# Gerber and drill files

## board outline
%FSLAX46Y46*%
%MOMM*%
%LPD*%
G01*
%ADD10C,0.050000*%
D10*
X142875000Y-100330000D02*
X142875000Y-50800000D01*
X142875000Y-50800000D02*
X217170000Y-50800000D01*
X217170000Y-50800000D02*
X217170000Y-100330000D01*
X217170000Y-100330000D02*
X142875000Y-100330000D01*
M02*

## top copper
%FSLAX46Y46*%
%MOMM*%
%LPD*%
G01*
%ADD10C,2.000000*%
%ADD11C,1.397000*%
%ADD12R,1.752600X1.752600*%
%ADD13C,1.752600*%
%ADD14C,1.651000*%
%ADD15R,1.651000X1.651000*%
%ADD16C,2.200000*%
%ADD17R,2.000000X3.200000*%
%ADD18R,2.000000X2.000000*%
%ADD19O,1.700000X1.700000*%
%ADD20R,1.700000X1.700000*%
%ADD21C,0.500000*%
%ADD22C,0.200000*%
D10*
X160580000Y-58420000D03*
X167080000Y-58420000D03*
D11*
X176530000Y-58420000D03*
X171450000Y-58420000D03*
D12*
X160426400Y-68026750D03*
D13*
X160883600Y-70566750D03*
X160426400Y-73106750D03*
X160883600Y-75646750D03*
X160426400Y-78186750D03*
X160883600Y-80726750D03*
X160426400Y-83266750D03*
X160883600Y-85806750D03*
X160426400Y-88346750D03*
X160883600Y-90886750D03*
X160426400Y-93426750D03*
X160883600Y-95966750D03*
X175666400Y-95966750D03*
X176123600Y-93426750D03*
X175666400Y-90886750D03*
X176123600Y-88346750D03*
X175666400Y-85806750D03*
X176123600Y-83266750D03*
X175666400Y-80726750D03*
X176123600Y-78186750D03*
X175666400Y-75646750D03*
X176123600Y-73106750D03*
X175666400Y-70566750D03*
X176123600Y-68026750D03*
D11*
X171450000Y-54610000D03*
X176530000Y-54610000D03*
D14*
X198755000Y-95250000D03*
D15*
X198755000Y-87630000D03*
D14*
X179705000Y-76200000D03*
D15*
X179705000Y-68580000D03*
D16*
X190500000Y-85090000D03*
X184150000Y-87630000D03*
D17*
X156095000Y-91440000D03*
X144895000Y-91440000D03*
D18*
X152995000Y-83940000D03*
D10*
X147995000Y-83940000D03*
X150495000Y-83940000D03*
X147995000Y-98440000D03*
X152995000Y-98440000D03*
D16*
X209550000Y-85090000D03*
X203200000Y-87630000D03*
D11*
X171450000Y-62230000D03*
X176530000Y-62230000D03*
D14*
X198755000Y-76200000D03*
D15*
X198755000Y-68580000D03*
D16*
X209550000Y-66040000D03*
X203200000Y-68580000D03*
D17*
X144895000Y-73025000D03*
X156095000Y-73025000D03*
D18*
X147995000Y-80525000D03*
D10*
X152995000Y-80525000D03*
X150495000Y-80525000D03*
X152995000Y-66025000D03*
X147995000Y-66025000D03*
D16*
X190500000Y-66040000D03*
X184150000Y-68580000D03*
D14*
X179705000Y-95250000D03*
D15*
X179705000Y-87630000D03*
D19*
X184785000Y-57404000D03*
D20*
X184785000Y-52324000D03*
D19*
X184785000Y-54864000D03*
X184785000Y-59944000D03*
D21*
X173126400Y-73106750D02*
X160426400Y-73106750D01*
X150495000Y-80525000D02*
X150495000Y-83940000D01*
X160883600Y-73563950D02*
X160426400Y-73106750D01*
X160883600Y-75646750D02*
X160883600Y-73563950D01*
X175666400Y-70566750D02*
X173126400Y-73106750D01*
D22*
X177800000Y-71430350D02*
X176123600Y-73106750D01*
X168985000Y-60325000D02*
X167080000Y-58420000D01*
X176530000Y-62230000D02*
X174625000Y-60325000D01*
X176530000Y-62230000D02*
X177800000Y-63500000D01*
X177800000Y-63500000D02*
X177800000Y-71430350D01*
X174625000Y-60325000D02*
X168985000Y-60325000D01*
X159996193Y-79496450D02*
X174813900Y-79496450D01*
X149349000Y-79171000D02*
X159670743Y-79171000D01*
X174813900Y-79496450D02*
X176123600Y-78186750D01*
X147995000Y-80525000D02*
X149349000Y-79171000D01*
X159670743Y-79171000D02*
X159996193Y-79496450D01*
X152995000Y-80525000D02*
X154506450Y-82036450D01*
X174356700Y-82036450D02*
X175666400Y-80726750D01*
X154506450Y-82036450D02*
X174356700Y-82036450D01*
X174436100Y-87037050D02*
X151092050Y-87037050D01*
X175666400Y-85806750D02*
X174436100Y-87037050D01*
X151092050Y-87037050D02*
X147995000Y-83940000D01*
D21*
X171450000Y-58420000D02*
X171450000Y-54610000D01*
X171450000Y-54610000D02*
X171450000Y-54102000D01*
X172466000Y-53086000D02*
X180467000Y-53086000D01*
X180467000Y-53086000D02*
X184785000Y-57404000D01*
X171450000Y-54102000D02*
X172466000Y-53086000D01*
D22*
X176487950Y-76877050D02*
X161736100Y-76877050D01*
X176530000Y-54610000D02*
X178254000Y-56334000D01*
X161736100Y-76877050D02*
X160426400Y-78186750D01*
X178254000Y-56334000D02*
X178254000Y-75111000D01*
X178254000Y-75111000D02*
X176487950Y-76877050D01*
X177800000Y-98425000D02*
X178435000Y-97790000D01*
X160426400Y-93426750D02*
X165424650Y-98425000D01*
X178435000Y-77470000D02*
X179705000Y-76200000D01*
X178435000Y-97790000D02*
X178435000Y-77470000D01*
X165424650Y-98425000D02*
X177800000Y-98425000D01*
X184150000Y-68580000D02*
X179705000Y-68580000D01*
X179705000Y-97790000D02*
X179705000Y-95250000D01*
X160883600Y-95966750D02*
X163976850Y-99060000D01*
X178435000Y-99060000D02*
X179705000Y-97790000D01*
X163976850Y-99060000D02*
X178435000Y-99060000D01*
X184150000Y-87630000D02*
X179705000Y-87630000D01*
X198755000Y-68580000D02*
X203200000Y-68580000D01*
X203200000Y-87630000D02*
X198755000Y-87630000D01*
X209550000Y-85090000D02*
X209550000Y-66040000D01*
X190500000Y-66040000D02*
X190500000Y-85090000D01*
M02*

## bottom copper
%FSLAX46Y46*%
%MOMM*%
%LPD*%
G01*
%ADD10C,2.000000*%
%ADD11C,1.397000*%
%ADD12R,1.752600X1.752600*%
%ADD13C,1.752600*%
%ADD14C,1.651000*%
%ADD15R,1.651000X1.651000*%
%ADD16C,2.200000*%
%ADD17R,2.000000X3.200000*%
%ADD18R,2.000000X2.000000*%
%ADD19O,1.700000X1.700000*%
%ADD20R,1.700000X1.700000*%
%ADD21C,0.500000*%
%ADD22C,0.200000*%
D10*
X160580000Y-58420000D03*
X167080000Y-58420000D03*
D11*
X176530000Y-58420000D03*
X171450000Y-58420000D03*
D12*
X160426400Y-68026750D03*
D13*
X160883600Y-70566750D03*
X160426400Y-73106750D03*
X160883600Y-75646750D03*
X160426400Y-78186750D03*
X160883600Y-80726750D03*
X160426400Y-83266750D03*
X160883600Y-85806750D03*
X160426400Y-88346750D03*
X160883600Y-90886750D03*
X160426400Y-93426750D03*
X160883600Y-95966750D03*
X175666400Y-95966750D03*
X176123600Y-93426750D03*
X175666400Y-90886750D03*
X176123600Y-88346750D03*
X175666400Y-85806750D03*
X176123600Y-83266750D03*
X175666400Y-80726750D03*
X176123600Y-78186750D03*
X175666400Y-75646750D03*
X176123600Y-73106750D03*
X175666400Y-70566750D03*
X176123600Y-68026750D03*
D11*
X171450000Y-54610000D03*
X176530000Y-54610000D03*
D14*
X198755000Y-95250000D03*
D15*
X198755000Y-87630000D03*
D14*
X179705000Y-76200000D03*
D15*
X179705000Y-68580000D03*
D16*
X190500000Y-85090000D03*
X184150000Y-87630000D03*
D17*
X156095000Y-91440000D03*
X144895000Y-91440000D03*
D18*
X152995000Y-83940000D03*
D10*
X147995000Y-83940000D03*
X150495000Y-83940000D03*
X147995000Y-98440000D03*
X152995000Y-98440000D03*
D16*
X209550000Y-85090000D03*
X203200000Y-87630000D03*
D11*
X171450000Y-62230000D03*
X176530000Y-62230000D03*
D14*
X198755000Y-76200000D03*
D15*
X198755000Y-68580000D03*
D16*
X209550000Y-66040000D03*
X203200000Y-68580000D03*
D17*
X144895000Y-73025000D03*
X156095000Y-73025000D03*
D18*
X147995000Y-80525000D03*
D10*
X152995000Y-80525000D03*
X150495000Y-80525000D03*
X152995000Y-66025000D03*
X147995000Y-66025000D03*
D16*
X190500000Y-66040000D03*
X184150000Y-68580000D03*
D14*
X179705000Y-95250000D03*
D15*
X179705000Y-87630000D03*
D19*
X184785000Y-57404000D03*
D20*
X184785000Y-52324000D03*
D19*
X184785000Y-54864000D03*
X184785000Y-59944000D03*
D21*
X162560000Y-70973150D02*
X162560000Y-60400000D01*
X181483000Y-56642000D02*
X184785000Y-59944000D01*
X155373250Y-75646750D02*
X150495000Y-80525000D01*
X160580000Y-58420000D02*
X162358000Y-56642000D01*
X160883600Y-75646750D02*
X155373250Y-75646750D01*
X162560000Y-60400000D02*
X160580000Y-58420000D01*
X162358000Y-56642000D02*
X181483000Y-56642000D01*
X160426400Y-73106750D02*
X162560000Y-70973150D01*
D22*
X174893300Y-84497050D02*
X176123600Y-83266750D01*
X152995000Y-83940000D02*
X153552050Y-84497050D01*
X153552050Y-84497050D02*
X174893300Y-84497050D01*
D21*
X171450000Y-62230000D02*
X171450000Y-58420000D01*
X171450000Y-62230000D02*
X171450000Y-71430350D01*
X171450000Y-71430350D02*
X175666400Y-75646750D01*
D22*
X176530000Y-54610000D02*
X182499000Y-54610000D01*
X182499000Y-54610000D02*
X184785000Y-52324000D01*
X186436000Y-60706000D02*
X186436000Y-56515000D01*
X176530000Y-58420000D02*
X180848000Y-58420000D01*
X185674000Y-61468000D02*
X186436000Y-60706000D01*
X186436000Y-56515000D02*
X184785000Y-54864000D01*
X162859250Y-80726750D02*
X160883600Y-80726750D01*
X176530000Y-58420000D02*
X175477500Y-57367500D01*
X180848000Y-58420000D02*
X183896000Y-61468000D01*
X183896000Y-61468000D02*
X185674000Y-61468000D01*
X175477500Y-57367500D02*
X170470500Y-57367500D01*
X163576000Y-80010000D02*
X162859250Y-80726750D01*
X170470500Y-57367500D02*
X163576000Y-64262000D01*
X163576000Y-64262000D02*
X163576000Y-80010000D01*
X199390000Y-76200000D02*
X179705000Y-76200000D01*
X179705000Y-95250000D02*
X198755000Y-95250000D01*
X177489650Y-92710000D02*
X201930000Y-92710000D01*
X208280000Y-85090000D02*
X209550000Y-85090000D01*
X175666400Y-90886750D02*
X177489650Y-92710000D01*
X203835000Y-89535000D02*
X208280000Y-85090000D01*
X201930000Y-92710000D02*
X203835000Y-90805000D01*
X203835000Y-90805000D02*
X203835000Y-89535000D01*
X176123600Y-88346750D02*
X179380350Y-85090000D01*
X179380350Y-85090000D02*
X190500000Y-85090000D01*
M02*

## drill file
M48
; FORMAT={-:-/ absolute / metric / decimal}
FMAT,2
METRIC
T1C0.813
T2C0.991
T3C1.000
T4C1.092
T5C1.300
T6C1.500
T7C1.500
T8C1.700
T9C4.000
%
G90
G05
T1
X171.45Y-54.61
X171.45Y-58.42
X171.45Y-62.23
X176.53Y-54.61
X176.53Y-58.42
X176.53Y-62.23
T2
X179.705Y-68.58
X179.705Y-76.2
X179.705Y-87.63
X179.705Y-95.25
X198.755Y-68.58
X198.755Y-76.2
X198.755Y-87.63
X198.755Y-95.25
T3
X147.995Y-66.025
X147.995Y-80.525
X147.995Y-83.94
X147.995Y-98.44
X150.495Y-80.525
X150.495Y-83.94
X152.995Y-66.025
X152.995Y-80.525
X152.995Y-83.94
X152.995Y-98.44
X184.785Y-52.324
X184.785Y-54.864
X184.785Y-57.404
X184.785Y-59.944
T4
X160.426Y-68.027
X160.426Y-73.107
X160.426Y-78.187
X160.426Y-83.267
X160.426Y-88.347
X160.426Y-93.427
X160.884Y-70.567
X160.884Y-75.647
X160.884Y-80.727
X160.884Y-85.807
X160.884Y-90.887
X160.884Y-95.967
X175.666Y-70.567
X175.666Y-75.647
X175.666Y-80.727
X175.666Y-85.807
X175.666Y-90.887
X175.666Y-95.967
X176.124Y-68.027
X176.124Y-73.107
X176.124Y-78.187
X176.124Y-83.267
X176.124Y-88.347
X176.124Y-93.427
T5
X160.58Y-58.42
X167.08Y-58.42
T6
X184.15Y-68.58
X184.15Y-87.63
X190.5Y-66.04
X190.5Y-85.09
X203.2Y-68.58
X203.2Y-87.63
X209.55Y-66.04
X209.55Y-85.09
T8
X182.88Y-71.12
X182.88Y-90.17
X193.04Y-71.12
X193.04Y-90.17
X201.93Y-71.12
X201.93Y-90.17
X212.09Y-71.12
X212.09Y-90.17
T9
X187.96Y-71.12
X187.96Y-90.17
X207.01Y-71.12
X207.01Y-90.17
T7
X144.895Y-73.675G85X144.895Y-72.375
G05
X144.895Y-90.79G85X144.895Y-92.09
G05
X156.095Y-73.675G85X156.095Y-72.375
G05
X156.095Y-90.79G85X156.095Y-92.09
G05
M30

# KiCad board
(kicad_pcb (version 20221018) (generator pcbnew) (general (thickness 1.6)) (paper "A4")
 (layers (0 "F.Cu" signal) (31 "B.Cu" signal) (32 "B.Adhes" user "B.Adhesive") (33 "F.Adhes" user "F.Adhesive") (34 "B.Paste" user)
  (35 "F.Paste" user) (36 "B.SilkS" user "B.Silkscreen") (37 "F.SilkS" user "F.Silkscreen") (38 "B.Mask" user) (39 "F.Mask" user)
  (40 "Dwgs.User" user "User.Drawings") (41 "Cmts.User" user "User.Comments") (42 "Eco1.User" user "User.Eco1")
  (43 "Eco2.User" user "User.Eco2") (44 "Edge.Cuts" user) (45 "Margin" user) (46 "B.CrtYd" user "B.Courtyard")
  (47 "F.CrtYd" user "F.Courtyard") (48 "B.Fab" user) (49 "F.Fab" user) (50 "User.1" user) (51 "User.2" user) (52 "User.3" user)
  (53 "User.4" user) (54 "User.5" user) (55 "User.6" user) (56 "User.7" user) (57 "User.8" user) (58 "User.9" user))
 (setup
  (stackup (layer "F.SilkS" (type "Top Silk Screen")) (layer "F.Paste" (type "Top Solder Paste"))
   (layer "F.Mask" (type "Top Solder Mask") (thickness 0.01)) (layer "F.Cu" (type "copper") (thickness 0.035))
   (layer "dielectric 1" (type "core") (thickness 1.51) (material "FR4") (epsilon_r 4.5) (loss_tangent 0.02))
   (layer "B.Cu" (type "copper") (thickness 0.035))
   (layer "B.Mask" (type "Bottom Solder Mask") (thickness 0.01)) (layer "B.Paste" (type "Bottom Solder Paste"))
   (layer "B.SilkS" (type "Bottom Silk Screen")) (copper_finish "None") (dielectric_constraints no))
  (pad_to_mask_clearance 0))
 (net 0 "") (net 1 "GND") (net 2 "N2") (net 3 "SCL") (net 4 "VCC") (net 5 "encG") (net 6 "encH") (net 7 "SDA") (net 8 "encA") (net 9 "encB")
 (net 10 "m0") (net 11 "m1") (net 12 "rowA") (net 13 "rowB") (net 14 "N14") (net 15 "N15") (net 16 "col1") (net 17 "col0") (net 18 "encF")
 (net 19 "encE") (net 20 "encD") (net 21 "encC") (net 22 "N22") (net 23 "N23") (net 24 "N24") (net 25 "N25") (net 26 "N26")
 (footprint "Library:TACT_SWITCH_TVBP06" (layer "F.Cu") (at 163.83 58.42)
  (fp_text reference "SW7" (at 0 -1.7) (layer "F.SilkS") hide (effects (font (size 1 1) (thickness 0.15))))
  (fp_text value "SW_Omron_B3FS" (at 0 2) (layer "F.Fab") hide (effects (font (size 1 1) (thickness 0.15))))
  (pad "1" thru_hole circle (at -3.25 0) (size 2 2) (drill 1.3) (layers "*.Cu" "*.Mask") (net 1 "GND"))
  (pad "2" thru_hole circle (at 3.25 0) (size 2 2) (drill 1.3) (layers "*.Cu" "*.Mask") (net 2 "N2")))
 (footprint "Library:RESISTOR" (layer "F.Cu") (at 173.99 58.42 180)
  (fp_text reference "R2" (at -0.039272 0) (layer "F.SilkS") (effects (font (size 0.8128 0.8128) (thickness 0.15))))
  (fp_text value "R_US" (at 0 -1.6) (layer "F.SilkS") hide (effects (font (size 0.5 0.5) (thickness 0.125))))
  (pad "1" thru_hole circle (at -2.54 0 180) (size 1.397 1.397) (drill 0.8128) (layers "*.Cu" "*.Mask") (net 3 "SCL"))
  (pad "2" thru_hole circle (at 2.54 0 180) (size 1.397 1.397) (drill 0.8128) (layers "*.Cu" "*.Mask") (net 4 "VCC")))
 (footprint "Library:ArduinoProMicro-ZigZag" (layer "F.Cu") (at 168.275 81.99675 -90)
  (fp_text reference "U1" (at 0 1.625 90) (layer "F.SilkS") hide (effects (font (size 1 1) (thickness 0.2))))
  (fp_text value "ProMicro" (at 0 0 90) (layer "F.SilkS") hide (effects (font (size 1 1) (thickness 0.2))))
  (pad "1" thru_hole rect (at -13.97 7.8486 270) (size 1.7526 1.7526) (drill 1.0922) (layers "*.Cu" "*.SilkS" "*.Mask") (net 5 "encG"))
  (pad "2" thru_hole circle (at -11.43 7.3914 270) (size 1.7526 1.7526) (drill 1.0922) (layers "*.Cu" "*.SilkS" "*.Mask") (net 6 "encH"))
  (pad "3" thru_hole circle (at -8.89 7.8486 270) (size 1.7526 1.7526) (drill 1.0922) (layers "*.Cu" "*.SilkS" "*.Mask") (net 1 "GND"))
  (pad "4" thru_hole circle (at -6.35 7.3914 270) (size 1.7526 1.7526) (drill 1.0922) (layers "*.Cu" "*.SilkS" "*.Mask") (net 1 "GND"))
  (pad "5" thru_hole circle (at -3.81 7.8486 270) (size 1.7526 1.7526) (drill 1.0922) (layers "*.Cu" "*.SilkS" "*.Mask") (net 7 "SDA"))
  (pad "6" thru_hole circle (at -1.27 7.3914 270) (size 1.7526 1.7526) (drill 1.0922) (layers "*.Cu" "*.SilkS" "*.Mask") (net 3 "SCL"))
  (pad "7" thru_hole circle (at 1.27 7.8486 270) (size 1.7526 1.7526) (drill 1.0922) (layers "*.Cu" "*.SilkS" "*.Mask") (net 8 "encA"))
  (pad "8" thru_hole circle (at 3.81 7.3914 270) (size 1.7526 1.7526) (drill 1.0922) (layers "*.Cu" "*.SilkS" "*.Mask") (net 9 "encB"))
  (pad "9" thru_hole circle (at 6.35 7.8486 270) (size 1.7526 1.7526) (drill 1.0922) (layers "*.Cu" "*.SilkS" "*.Mask") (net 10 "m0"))
  (pad "10" thru_hole circle (at 8.89 7.3914 270) (size 1.7526 1.7526) (drill 1.0922) (layers "*.Cu" "*.SilkS" "*.Mask") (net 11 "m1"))
  (pad "11" thru_hole circle (at 11.43 7.8486 270) (size 1.7526 1.7526) (drill 1.0922) (layers "*.Cu" "*.SilkS" "*.Mask") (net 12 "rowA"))
  (pad "12" thru_hole circle (at 13.97 7.3914 270) (size 1.7526 1.7526) (drill 1.0922) (layers "*.Cu" "*.SilkS" "*.Mask") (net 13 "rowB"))
  (pad "13" thru_hole circle (at 13.97 -7.3914 270) (size 1.7526 1.7526) (drill 1.0922) (layers "*.Cu" "*.SilkS" "*.Mask") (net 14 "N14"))
  (pad "14" thru_hole circle (at 11.43 -7.8486 270) (size 1.7526 1.7526) (drill 1.0922) (layers "*.Cu" "*.SilkS" "*.Mask") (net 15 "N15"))
  (pad "15" thru_hole circle (at 8.89 -7.3914 270) (size 1.7526 1.7526) (drill 1.0922) (layers "*.Cu" "*.SilkS" "*.Mask") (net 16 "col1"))
  (pad "16" thru_hole circle (at 6.35 -7.8486 270) (size 1.7526 1.7526) (drill 1.0922) (layers "*.Cu" "*.SilkS" "*.Mask") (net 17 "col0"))
  (pad "17" thru_hole circle (at 3.81 -7.3914 270) (size 1.7526 1.7526) (drill 1.0922) (layers "*.Cu" "*.SilkS" "*.Mask") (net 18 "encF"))
  (pad "18" thru_hole circle (at 1.27 -7.8486 270) (size 1.7526 1.7526) (drill 1.0922) (layers "*.Cu" "*.SilkS" "*.Mask") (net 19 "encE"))
  (pad "19" thru_hole circle (at -1.27 -7.3914 270) (size 1.7526 1.7526) (drill 1.0922) (layers "*.Cu" "*.SilkS" "*.Mask") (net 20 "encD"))
  (pad "20" thru_hole circle (at -3.81 -7.8486 270) (size 1.7526 1.7526) (drill 1.0922) (layers "*.Cu" "*.SilkS" "*.Mask") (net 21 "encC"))
  (pad "21" thru_hole circle (at -6.35 -7.3914 270) (size 1.7526 1.7526) (drill 1.0922) (layers "*.Cu" "*.SilkS" "*.Mask") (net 4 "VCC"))
  (pad "22" thru_hole circle (at -8.89 -7.8486 270) (size 1.7526 1.7526) (drill 1.0922) (layers "*.Cu" "*.SilkS" "*.Mask") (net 2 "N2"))
  (pad "23" thru_hole circle (at -11.43 -7.3914 270) (size 1.7526 1.7526) (drill 1.0922) (layers "*.Cu" "*.SilkS" "*.Mask") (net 1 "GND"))
  (pad "24" thru_hole circle (at -13.97 -7.8486 270) (size 1.7526 1.7526) (drill 1.0922) (layers "*.Cu" "*.SilkS" "*.Mask") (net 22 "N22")))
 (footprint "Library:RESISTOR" (layer "F.Cu") (at 173.99 54.61)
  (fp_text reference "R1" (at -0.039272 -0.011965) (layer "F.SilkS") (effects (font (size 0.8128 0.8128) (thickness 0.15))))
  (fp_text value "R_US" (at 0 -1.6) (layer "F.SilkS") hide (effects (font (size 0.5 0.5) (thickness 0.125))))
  (pad "1" thru_hole circle (at -2.54 0) (size 1.397 1.397) (drill 0.8128) (layers "*.Cu" "*.Mask") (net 4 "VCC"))
  (pad "2" thru_hole circle (at 2.54 0) (size 1.397 1.397) (drill 0.8128) (layers "*.Cu" "*.Mask") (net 7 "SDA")))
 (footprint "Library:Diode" (layer "F.Cu") (at 198.755 91.44 90)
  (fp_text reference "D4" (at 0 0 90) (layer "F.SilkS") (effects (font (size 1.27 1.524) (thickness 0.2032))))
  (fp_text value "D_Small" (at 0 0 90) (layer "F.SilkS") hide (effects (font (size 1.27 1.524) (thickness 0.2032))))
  (pad "1" thru_hole circle (at -3.81 0 90) (size 1.651 1.651) (drill 0.9906) (layers "*.Cu" "*.SilkS" "*.Mask") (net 13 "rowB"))
  (pad "2" thru_hole rect (at 3.81 0 90) (size 1.651 1.651) (drill 0.9906) (layers "*.Cu" "*.SilkS" "*.Mask") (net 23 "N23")))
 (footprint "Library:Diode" (layer "F.Cu") (at 179.705 72.39 90)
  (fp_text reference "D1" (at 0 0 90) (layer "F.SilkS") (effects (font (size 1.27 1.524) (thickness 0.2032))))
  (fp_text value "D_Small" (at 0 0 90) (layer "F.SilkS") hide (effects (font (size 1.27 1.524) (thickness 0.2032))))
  (pad "1" thru_hole circle (at -3.81 0 90) (size 1.651 1.651) (drill 0.9906) (layers "*.Cu" "*.SilkS" "*.Mask") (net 12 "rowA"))
  (pad "2" thru_hole rect (at 3.81 0 90) (size 1.651 1.651) (drill 0.9906) (layers "*.Cu" "*.SilkS" "*.Mask") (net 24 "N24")))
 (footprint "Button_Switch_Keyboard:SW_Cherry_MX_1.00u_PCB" (layer "F.Cu") (at 190.5 85.09)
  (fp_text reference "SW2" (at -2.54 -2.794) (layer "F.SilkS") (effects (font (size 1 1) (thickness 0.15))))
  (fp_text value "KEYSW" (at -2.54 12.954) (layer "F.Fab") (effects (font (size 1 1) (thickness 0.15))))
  (pad "" np_thru_hole circle (at -7.62 5.08) (size 1.7 1.7) (drill 1.7) (layers "*.Cu" "*.Mask"))
  (pad "" np_thru_hole circle (at -2.54 5.08) (size 4 4) (drill 4) (layers "*.Cu" "*.Mask"))
  (pad "" np_thru_hole circle (at 2.54 5.08) (size 1.7 1.7) (drill 1.7) (layers "*.Cu" "*.Mask"))
  (pad "1" thru_hole circle (at 0 0) (size 2.2 2.2) (drill 1.5) (layers "*.Cu" "*.Mask") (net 17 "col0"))
  (pad "2" thru_hole circle (at -6.35 2.54) (size 2.2 2.2) (drill 1.5) (layers "*.Cu" "*.Mask") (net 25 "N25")))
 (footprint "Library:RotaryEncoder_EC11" (layer "F.Cu") (at 150.495 91.44 -90)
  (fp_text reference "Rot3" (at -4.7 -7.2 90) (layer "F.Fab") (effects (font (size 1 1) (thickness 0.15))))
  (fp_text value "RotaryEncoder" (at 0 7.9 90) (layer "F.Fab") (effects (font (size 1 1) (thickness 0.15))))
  (pad "" np_thru_hole rect (at 0 -5.6 270) (size 3.2 2) (drill oval 2.8 1.5) (layers "*.Cu" "*.Mask"))
  (pad "" np_thru_hole rect (at 0 5.6 270) (size 3.2 2) (drill oval 2.8 1.5) (layers "*.Cu" "*.Mask"))
  (pad "A" thru_hole rect (at -7.5 -2.5 270) (size 2 2) (drill 1) (layers "*.Cu" "*.Mask") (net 19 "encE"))
  (pad "B" thru_hole circle (at -7.5 2.5 270) (size 2 2) (drill 1) (layers "*.Cu" "*.Mask") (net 18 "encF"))
  (pad "C" thru_hole circle (at -7.5 0 270) (size 2 2) (drill 1) (layers "*.Cu" "*.Mask") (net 1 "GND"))
  (pad "S1" thru_hole circle (at 7 2.5 270) (size 2 2) (drill 1) (layers "*.Cu" "*.Mask"))
  (pad "S2" thru_hole circle (at 7 -2.5 270) (size 2 2) (drill 1) (layers "*.Cu" "*.Mask")))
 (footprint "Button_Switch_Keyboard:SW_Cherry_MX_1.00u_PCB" (layer "F.Cu") (at 209.55 85.09)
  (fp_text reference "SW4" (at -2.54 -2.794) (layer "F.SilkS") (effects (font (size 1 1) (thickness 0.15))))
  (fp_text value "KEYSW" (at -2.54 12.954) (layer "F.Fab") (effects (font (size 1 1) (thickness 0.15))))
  (pad "" np_thru_hole circle (at -7.62 5.08) (size 1.7 1.7) (drill 1.7) (layers "*.Cu" "*.Mask"))
  (pad "" np_thru_hole circle (at -2.54 5.08) (size 4 4) (drill 4) (layers "*.Cu" "*.Mask"))
  (pad "" np_thru_hole circle (at 2.54 5.08) (size 1.7 1.7) (drill 1.7) (layers "*.Cu" "*.Mask"))
  (pad "1" thru_hole circle (at 0 0) (size 2.2 2.2) (drill 1.5) (layers "*.Cu" "*.Mask") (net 16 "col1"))
  (pad "2" thru_hole circle (at -6.35 2.54) (size 2.2 2.2) (drill 1.5) (layers "*.Cu" "*.Mask") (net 23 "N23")))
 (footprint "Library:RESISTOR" (layer "F.Cu") (at 173.99 62.23)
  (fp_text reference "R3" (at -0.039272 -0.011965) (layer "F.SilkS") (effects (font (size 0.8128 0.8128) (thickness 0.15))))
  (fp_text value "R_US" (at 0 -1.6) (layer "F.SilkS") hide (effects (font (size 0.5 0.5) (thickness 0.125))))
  (pad "1" thru_hole circle (at -2.54 0) (size 1.397 1.397) (drill 0.8128) (layers "*.Cu" "*.Mask") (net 4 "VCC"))
  (pad "2" thru_hole circle (at 2.54 0) (size 1.397 1.397) (drill 0.8128) (layers "*.Cu" "*.Mask") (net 2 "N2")))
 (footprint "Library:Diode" (layer "F.Cu") (at 198.755 72.39 90)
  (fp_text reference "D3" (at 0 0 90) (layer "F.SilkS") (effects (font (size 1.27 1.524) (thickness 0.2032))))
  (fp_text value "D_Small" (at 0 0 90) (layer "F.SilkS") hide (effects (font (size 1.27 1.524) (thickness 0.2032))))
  (pad "1" thru_hole circle (at -3.81 0 90) (size 1.651 1.651) (drill 0.9906) (layers "*.Cu" "*.SilkS" "*.Mask") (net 12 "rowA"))
  (pad "2" thru_hole rect (at 3.81 0 90) (size 1.651 1.651) (drill 0.9906) (layers "*.Cu" "*.SilkS" "*.Mask") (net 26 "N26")))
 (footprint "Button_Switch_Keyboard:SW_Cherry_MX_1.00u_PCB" (layer "F.Cu") (at 209.55 66.04)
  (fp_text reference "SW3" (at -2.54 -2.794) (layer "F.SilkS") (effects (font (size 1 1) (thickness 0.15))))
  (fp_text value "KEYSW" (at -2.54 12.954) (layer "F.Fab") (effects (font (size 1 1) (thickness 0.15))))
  (pad "" np_thru_hole circle (at -7.62 5.08) (size 1.7 1.7) (drill 1.7) (layers "*.Cu" "*.Mask"))
  (pad "" np_thru_hole circle (at -2.54 5.08) (size 4 4) (drill 4) (layers "*.Cu" "*.Mask"))
  (pad "" np_thru_hole circle (at 2.54 5.08) (size 1.7 1.7) (drill 1.7) (layers "*.Cu" "*.Mask"))
  (pad "1" thru_hole circle (at 0 0) (size 2.2 2.2) (drill 1.5) (layers "*.Cu" "*.Mask") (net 16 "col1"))
  (pad "2" thru_hole circle (at -6.35 2.54) (size 2.2 2.2) (drill 1.5) (layers "*.Cu" "*.Mask") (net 26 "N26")))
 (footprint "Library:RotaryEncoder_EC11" (layer "F.Cu") (at 150.495 73.025 90)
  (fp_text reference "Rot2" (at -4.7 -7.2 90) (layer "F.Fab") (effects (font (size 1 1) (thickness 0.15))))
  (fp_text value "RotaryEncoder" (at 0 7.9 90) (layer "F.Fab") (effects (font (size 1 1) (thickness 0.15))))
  (pad "" np_thru_hole rect (at 0 -5.6 90) (size 3.2 2) (drill oval 2.8 1.5) (layers "*.Cu" "*.Mask"))
  (pad "" np_thru_hole rect (at 0 5.6 90) (size 3.2 2) (drill oval 2.8 1.5) (layers "*.Cu" "*.Mask"))
  (pad "A" thru_hole rect (at -7.5 -2.5 90) (size 2 2) (drill 1) (layers "*.Cu" "*.Mask") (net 21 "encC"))
  (pad "B" thru_hole circle (at -7.5 2.5 90) (size 2 2) (drill 1) (layers "*.Cu" "*.Mask") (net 20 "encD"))
  (pad "C" thru_hole circle (at -7.5 0 90) (size 2 2) (drill 1) (layers "*.Cu" "*.Mask") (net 1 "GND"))
  (pad "S1" thru_hole circle (at 7 2.5 90) (size 2 2) (drill 1) (layers "*.Cu" "*.Mask"))
  (pad "S2" thru_hole circle (at 7 -2.5 90) (size 2 2) (drill 1) (layers "*.Cu" "*.Mask")))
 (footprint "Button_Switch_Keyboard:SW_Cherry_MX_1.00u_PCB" (layer "F.Cu") (at 190.5 66.04)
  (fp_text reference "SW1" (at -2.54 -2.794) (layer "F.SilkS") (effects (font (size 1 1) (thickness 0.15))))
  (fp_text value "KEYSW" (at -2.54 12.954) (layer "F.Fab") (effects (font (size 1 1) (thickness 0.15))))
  (pad "" np_thru_hole circle (at -7.62 5.08) (size 1.7 1.7) (drill 1.7) (layers "*.Cu" "*.Mask"))
  (pad "" np_thru_hole circle (at -2.54 5.08) (size 4 4) (drill 4) (layers "*.Cu" "*.Mask"))
  (pad "" np_thru_hole circle (at 2.54 5.08) (size 1.7 1.7) (drill 1.7) (layers "*.Cu" "*.Mask"))
  (pad "1" thru_hole circle (at 0 0) (size 2.2 2.2) (drill 1.5) (layers "*.Cu" "*.Mask") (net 17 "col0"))
  (pad "2" thru_hole circle (at -6.35 2.54) (size 2.2 2.2) (drill 1.5) (layers "*.Cu" "*.Mask") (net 24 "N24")))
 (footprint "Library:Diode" (layer "F.Cu") (at 179.705 91.44 90)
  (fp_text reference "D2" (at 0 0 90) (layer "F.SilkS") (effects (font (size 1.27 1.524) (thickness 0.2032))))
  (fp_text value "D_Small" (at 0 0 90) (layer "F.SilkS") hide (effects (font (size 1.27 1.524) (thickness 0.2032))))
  (pad "1" thru_hole circle (at -3.81 0 90) (size 1.651 1.651) (drill 0.9906) (layers "*.Cu" "*.SilkS" "*.Mask") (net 13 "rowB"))
  (pad "2" thru_hole rect (at 3.81 0 90) (size 1.651 1.651) (drill 0.9906) (layers "*.Cu" "*.SilkS" "*.Mask") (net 25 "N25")))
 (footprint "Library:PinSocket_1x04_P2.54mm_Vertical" (layer "F.Cu") (at 184.785 52.324)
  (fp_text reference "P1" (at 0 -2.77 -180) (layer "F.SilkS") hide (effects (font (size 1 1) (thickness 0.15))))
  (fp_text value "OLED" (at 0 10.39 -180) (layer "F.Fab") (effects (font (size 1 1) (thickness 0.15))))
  (pad "" thru_hole oval (at 0 5.08) (size 1.7 1.7) (drill 1) (layers "*.Cu" "*.Mask") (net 4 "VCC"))
  (pad "1" thru_hole rect (at 0 0) (size 1.7 1.7) (drill 1) (layers "*.Cu" "*.Mask") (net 7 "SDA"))
  (pad "2" thru_hole oval (at 0 2.54) (size 1.7 1.7) (drill 1) (layers "*.Cu" "*.Mask") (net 3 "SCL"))
  (pad "4" thru_hole oval (at 0 7.62) (size 1.7 1.7) (drill 1) (layers "*.Cu" "*.Mask") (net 1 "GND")))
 (gr_line (start 142.875 100.33) (end 142.875 50.8) (stroke (width 0.05) (type default)) (layer "Edge.Cuts"))
 (gr_line (start 142.875 50.8) (end 217.17 50.8) (stroke (width 0.05) (type default)) (layer "Edge.Cuts"))
 (gr_line (start 217.17 50.8) (end 217.17 100.33) (stroke (width 0.05) (type default)) (layer "Edge.Cuts"))
 (gr_line (start 217.17 100.33) (end 142.875 100.33) (stroke (width 0.05) (type default)) (layer "Edge.Cuts"))
 (segment (start 173.1264 73.10675) (end 160.4264 73.10675) (width 0.5) (layer "F.Cu") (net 1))
 (segment (start 150.495 80.525) (end 150.495 83.94) (width 0.5) (layer "F.Cu") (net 1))
 (segment (start 160.8836 73.56395) (end 160.4264 73.10675) (width 0.5) (layer "F.Cu") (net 1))
 (segment (start 160.8836 75.64675) (end 160.8836 73.56395) (width 0.5) (layer "F.Cu") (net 1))
 (segment (start 175.6664 70.56675) (end 173.1264 73.10675) (width 0.5) (layer "F.Cu") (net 1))
 (segment (start 162.56 70.97315) (end 162.56 60.4) (width 0.5) (layer "B.Cu") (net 1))
 (segment (start 181.483 56.642) (end 184.785 59.944) (width 0.5) (layer "B.Cu") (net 1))
 (segment (start 155.37325 75.64675) (end 150.495 80.525) (width 0.5) (layer "B.Cu") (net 1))
 (segment (start 160.58 58.42) (end 162.358 56.642) (width 0.5) (layer "B.Cu") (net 1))
 (segment (start 160.8836 75.64675) (end 155.37325 75.64675) (width 0.5) (layer "B.Cu") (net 1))
 (segment (start 162.56 60.4) (end 160.58 58.42) (width 0.5) (layer "B.Cu") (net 1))
 (segment (start 162.358 56.642) (end 181.483 56.642) (width 0.5) (layer "B.Cu") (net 1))
 (segment (start 160.4264 73.10675) (end 162.56 70.97315) (width 0.5) (layer "B.Cu") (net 1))
 (segment (start 177.8 71.43035) (end 176.1236 73.10675) (width 0.2) (layer "F.Cu") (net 2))
 (segment (start 168.985 60.325) (end 167.08 58.42) (width 0.2) (layer "F.Cu") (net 2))
 (segment (start 176.53 62.23) (end 174.625 60.325) (width 0.2) (layer "F.Cu") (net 2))
 (segment (start 176.53 62.23) (end 177.8 63.5) (width 0.2) (layer "F.Cu") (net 2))
 (segment (start 177.8 63.5) (end 177.8 71.43035) (width 0.2) (layer "F.Cu") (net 2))
 (segment (start 174.625 60.325) (end 168.985 60.325) (width 0.2) (layer "F.Cu") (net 2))
 (segment (start 159.996193 79.49645) (end 174.8139 79.49645) (width 0.2) (layer "F.Cu") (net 21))
 (segment (start 149.349 79.171) (end 159.670743 79.171) (width 0.2) (layer "F.Cu") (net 21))
 (segment (start 174.8139 79.49645) (end 176.1236 78.18675) (width 0.2) (layer "F.Cu") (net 21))
 (segment (start 147.995 80.525) (end 149.349 79.171) (width 0.2) (layer "F.Cu") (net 21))
 (segment (start 159.670743 79.171) (end 159.996193 79.49645) (width 0.2) (layer "F.Cu") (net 21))
 (segment (start 152.995 80.525) (end 154.50645 82.03645) (width 0.2) (layer "F.Cu") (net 20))
 (segment (start 174.3567 82.03645) (end 175.6664 80.72675) (width 0.2) (layer "F.Cu") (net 20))
 (segment (start 154.50645 82.03645) (end 174.3567 82.03645) (width 0.2) (layer "F.Cu") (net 20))
 (segment (start 174.8933 84.49705) (end 176.1236 83.26675) (width 0.2) (layer "B.Cu") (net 19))
 (segment (start 152.995 83.94) (end 153.55205 84.49705) (width 0.2) (layer "B.Cu") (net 19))
 (segment (start 153.55205 84.49705) (end 174.8933 84.49705) (width 0.2) (layer "B.Cu") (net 19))
 (segment (start 174.4361 87.03705) (end 151.09205 87.03705) (width 0.2) (layer "F.Cu") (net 18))
 (segment (start 175.6664 85.80675) (end 174.4361 87.03705) (width 0.2) (layer "F.Cu") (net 18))
 (segment (start 151.09205 87.03705) (end 147.995 83.94) (width 0.2) (layer "F.Cu") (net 18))
 (segment (start 171.45 58.42) (end 171.45 54.61) (width 0.5) (layer "F.Cu") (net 4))
 (segment (start 171.45 54.61) (end 171.45 54.102) (width 0.5) (layer "F.Cu") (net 4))
 (segment (start 172.466 53.086) (end 180.467 53.086) (width 0.5) (layer "F.Cu") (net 4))
 (segment (start 180.467 53.086) (end 184.785 57.404) (width 0.5) (layer "F.Cu") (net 4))
 (segment (start 171.45 54.102) (end 172.466 53.086) (width 0.5) (layer "F.Cu") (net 4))
 (segment (start 171.45 62.23) (end 171.45 58.42) (width 0.5) (layer "B.Cu") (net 4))
 (segment (start 171.45 62.23) (end 171.45 71.43035) (width 0.5) (layer "B.Cu") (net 4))
 (segment (start 171.45 71.43035) (end 175.6664 75.64675) (width 0.5) (layer "B.Cu") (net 4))
 (segment (start 176.48795 76.87705) (end 161.7361 76.87705) (width 0.2) (layer "F.Cu") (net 7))
 (segment (start 176.53 54.61) (end 178.254 56.334) (width 0.2) (layer "F.Cu") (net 7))
 (segment (start 161.7361 76.87705) (end 160.4264 78.18675) (width 0.2) (layer "F.Cu") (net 7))
 (segment (start 178.254 56.334) (end 178.254 75.111) (width 0.2) (layer "F.Cu") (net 7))
 (segment (start 178.254 75.111) (end 176.48795 76.87705) (width 0.2) (layer "F.Cu") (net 7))
 (segment (start 176.53 54.61) (end 182.499 54.61) (width 0.2) (layer "B.Cu") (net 7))
 (segment (start 182.499 54.61) (end 184.785 52.324) (width 0.2) (layer "B.Cu") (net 7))
 (segment (start 186.436 60.706) (end 186.436 56.515) (width 0.2) (layer "B.Cu") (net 3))
 (segment (start 176.53 58.42) (end 180.848 58.42) (width 0.2) (layer "B.Cu") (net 3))
 (segment (start 185.674 61.468) (end 186.436 60.706) (width 0.2) (layer "B.Cu") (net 3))
 (segment (start 186.436 56.515) (end 184.785 54.864) (width 0.2) (layer "B.Cu") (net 3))
 (segment (start 162.85925 80.72675) (end 160.8836 80.72675) (width 0.2) (layer "B.Cu") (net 3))
 (segment (start 176.53 58.42) (end 175.4775 57.3675) (width 0.2) (layer "B.Cu") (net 3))
 (segment (start 180.848 58.42) (end 183.896 61.468) (width 0.2) (layer "B.Cu") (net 3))
 (segment (start 183.896 61.468) (end 185.674 61.468) (width 0.2) (layer "B.Cu") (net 3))
 (segment (start 175.4775 57.3675) (end 170.4705 57.3675) (width 0.2) (layer "B.Cu") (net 3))
 (segment (start 163.576 80.01) (end 162.85925 80.72675) (width 0.2) (layer "B.Cu") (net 3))
 (segment (start 170.4705 57.3675) (end 163.576 64.262) (width 0.2) (layer "B.Cu") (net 3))
 (segment (start 163.576 64.262) (end 163.576 80.01) (width 0.2) (layer "B.Cu") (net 3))
 (segment (start 177.8 98.425) (end 178.435 97.79) (width 0.2) (layer "F.Cu") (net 12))
 (segment (start 160.4264 93.42675) (end 165.42465 98.425) (width 0.2) (layer "F.Cu") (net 12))
 (segment (start 178.435 77.47) (end 179.705 76.2) (width 0.2) (layer "F.Cu") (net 12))
 (segment (start 178.435 97.79) (end 178.435 77.47) (width 0.2) (layer "F.Cu") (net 12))
 (segment (start 165.42465 98.425) (end 177.8 98.425) (width 0.2) (layer "F.Cu") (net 12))
 (segment (start 199.39 76.2) (end 179.705 76.2) (width 0.2) (layer "B.Cu") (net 12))
 (segment (start 184.15 68.58) (end 179.705 68.58) (width 0.2) (layer "F.Cu") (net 24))
 (segment (start 179.705 97.79) (end 179.705 95.25) (width 0.2) (layer "F.Cu") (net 13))
 (segment (start 160.8836 95.96675) (end 163.97685 99.06) (width 0.2) (layer "F.Cu") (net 13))
 (segment (start 178.435 99.06) (end 179.705 97.79) (width 0.2) (layer "F.Cu") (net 13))
 (segment (start 163.97685 99.06) (end 178.435 99.06) (width 0.2) (layer "F.Cu") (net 13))
 (segment (start 179.705 95.25) (end 198.755 95.25) (width 0.2) (layer "B.Cu") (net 13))
 (segment (start 184.15 87.63) (end 179.705 87.63) (width 0.2) (layer "F.Cu") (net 25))
 (segment (start 198.755 68.58) (end 203.2 68.58) (width 0.2) (layer "F.Cu") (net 26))
 (segment (start 203.2 87.63) (end 198.755 87.63) (width 0.2) (layer "F.Cu") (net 23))
 (segment (start 209.55 85.09) (end 209.55 66.04) (width 0.2) (layer "F.Cu") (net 16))
 (segment (start 177.48965 92.71) (end 201.93 92.71) (width 0.2) (layer "B.Cu") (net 16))
 (segment (start 208.28 85.09) (end 209.55 85.09) (width 0.2) (layer "B.Cu") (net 16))
 (segment (start 175.6664 90.88675) (end 177.48965 92.71) (width 0.2) (layer "B.Cu") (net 16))
 (segment (start 203.835 89.535) (end 208.28 85.09) (width 0.2) (layer "B.Cu") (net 16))
 (segment (start 201.93 92.71) (end 203.835 90.805) (width 0.2) (layer "B.Cu") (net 16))
 (segment (start 203.835 90.805) (end 203.835 89.535) (width 0.2) (layer "B.Cu") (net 16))
 (segment (start 190.5 66.04) (end 190.5 85.09) (width 0.2) (layer "F.Cu") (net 17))
 (segment (start 176.1236 88.34675) (end 179.38035 85.09) (width 0.2) (layer "B.Cu") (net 17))
 (segment (start 179.38035 85.09) (end 190.5 85.09) (width 0.2) (layer "B.Cu") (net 17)))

